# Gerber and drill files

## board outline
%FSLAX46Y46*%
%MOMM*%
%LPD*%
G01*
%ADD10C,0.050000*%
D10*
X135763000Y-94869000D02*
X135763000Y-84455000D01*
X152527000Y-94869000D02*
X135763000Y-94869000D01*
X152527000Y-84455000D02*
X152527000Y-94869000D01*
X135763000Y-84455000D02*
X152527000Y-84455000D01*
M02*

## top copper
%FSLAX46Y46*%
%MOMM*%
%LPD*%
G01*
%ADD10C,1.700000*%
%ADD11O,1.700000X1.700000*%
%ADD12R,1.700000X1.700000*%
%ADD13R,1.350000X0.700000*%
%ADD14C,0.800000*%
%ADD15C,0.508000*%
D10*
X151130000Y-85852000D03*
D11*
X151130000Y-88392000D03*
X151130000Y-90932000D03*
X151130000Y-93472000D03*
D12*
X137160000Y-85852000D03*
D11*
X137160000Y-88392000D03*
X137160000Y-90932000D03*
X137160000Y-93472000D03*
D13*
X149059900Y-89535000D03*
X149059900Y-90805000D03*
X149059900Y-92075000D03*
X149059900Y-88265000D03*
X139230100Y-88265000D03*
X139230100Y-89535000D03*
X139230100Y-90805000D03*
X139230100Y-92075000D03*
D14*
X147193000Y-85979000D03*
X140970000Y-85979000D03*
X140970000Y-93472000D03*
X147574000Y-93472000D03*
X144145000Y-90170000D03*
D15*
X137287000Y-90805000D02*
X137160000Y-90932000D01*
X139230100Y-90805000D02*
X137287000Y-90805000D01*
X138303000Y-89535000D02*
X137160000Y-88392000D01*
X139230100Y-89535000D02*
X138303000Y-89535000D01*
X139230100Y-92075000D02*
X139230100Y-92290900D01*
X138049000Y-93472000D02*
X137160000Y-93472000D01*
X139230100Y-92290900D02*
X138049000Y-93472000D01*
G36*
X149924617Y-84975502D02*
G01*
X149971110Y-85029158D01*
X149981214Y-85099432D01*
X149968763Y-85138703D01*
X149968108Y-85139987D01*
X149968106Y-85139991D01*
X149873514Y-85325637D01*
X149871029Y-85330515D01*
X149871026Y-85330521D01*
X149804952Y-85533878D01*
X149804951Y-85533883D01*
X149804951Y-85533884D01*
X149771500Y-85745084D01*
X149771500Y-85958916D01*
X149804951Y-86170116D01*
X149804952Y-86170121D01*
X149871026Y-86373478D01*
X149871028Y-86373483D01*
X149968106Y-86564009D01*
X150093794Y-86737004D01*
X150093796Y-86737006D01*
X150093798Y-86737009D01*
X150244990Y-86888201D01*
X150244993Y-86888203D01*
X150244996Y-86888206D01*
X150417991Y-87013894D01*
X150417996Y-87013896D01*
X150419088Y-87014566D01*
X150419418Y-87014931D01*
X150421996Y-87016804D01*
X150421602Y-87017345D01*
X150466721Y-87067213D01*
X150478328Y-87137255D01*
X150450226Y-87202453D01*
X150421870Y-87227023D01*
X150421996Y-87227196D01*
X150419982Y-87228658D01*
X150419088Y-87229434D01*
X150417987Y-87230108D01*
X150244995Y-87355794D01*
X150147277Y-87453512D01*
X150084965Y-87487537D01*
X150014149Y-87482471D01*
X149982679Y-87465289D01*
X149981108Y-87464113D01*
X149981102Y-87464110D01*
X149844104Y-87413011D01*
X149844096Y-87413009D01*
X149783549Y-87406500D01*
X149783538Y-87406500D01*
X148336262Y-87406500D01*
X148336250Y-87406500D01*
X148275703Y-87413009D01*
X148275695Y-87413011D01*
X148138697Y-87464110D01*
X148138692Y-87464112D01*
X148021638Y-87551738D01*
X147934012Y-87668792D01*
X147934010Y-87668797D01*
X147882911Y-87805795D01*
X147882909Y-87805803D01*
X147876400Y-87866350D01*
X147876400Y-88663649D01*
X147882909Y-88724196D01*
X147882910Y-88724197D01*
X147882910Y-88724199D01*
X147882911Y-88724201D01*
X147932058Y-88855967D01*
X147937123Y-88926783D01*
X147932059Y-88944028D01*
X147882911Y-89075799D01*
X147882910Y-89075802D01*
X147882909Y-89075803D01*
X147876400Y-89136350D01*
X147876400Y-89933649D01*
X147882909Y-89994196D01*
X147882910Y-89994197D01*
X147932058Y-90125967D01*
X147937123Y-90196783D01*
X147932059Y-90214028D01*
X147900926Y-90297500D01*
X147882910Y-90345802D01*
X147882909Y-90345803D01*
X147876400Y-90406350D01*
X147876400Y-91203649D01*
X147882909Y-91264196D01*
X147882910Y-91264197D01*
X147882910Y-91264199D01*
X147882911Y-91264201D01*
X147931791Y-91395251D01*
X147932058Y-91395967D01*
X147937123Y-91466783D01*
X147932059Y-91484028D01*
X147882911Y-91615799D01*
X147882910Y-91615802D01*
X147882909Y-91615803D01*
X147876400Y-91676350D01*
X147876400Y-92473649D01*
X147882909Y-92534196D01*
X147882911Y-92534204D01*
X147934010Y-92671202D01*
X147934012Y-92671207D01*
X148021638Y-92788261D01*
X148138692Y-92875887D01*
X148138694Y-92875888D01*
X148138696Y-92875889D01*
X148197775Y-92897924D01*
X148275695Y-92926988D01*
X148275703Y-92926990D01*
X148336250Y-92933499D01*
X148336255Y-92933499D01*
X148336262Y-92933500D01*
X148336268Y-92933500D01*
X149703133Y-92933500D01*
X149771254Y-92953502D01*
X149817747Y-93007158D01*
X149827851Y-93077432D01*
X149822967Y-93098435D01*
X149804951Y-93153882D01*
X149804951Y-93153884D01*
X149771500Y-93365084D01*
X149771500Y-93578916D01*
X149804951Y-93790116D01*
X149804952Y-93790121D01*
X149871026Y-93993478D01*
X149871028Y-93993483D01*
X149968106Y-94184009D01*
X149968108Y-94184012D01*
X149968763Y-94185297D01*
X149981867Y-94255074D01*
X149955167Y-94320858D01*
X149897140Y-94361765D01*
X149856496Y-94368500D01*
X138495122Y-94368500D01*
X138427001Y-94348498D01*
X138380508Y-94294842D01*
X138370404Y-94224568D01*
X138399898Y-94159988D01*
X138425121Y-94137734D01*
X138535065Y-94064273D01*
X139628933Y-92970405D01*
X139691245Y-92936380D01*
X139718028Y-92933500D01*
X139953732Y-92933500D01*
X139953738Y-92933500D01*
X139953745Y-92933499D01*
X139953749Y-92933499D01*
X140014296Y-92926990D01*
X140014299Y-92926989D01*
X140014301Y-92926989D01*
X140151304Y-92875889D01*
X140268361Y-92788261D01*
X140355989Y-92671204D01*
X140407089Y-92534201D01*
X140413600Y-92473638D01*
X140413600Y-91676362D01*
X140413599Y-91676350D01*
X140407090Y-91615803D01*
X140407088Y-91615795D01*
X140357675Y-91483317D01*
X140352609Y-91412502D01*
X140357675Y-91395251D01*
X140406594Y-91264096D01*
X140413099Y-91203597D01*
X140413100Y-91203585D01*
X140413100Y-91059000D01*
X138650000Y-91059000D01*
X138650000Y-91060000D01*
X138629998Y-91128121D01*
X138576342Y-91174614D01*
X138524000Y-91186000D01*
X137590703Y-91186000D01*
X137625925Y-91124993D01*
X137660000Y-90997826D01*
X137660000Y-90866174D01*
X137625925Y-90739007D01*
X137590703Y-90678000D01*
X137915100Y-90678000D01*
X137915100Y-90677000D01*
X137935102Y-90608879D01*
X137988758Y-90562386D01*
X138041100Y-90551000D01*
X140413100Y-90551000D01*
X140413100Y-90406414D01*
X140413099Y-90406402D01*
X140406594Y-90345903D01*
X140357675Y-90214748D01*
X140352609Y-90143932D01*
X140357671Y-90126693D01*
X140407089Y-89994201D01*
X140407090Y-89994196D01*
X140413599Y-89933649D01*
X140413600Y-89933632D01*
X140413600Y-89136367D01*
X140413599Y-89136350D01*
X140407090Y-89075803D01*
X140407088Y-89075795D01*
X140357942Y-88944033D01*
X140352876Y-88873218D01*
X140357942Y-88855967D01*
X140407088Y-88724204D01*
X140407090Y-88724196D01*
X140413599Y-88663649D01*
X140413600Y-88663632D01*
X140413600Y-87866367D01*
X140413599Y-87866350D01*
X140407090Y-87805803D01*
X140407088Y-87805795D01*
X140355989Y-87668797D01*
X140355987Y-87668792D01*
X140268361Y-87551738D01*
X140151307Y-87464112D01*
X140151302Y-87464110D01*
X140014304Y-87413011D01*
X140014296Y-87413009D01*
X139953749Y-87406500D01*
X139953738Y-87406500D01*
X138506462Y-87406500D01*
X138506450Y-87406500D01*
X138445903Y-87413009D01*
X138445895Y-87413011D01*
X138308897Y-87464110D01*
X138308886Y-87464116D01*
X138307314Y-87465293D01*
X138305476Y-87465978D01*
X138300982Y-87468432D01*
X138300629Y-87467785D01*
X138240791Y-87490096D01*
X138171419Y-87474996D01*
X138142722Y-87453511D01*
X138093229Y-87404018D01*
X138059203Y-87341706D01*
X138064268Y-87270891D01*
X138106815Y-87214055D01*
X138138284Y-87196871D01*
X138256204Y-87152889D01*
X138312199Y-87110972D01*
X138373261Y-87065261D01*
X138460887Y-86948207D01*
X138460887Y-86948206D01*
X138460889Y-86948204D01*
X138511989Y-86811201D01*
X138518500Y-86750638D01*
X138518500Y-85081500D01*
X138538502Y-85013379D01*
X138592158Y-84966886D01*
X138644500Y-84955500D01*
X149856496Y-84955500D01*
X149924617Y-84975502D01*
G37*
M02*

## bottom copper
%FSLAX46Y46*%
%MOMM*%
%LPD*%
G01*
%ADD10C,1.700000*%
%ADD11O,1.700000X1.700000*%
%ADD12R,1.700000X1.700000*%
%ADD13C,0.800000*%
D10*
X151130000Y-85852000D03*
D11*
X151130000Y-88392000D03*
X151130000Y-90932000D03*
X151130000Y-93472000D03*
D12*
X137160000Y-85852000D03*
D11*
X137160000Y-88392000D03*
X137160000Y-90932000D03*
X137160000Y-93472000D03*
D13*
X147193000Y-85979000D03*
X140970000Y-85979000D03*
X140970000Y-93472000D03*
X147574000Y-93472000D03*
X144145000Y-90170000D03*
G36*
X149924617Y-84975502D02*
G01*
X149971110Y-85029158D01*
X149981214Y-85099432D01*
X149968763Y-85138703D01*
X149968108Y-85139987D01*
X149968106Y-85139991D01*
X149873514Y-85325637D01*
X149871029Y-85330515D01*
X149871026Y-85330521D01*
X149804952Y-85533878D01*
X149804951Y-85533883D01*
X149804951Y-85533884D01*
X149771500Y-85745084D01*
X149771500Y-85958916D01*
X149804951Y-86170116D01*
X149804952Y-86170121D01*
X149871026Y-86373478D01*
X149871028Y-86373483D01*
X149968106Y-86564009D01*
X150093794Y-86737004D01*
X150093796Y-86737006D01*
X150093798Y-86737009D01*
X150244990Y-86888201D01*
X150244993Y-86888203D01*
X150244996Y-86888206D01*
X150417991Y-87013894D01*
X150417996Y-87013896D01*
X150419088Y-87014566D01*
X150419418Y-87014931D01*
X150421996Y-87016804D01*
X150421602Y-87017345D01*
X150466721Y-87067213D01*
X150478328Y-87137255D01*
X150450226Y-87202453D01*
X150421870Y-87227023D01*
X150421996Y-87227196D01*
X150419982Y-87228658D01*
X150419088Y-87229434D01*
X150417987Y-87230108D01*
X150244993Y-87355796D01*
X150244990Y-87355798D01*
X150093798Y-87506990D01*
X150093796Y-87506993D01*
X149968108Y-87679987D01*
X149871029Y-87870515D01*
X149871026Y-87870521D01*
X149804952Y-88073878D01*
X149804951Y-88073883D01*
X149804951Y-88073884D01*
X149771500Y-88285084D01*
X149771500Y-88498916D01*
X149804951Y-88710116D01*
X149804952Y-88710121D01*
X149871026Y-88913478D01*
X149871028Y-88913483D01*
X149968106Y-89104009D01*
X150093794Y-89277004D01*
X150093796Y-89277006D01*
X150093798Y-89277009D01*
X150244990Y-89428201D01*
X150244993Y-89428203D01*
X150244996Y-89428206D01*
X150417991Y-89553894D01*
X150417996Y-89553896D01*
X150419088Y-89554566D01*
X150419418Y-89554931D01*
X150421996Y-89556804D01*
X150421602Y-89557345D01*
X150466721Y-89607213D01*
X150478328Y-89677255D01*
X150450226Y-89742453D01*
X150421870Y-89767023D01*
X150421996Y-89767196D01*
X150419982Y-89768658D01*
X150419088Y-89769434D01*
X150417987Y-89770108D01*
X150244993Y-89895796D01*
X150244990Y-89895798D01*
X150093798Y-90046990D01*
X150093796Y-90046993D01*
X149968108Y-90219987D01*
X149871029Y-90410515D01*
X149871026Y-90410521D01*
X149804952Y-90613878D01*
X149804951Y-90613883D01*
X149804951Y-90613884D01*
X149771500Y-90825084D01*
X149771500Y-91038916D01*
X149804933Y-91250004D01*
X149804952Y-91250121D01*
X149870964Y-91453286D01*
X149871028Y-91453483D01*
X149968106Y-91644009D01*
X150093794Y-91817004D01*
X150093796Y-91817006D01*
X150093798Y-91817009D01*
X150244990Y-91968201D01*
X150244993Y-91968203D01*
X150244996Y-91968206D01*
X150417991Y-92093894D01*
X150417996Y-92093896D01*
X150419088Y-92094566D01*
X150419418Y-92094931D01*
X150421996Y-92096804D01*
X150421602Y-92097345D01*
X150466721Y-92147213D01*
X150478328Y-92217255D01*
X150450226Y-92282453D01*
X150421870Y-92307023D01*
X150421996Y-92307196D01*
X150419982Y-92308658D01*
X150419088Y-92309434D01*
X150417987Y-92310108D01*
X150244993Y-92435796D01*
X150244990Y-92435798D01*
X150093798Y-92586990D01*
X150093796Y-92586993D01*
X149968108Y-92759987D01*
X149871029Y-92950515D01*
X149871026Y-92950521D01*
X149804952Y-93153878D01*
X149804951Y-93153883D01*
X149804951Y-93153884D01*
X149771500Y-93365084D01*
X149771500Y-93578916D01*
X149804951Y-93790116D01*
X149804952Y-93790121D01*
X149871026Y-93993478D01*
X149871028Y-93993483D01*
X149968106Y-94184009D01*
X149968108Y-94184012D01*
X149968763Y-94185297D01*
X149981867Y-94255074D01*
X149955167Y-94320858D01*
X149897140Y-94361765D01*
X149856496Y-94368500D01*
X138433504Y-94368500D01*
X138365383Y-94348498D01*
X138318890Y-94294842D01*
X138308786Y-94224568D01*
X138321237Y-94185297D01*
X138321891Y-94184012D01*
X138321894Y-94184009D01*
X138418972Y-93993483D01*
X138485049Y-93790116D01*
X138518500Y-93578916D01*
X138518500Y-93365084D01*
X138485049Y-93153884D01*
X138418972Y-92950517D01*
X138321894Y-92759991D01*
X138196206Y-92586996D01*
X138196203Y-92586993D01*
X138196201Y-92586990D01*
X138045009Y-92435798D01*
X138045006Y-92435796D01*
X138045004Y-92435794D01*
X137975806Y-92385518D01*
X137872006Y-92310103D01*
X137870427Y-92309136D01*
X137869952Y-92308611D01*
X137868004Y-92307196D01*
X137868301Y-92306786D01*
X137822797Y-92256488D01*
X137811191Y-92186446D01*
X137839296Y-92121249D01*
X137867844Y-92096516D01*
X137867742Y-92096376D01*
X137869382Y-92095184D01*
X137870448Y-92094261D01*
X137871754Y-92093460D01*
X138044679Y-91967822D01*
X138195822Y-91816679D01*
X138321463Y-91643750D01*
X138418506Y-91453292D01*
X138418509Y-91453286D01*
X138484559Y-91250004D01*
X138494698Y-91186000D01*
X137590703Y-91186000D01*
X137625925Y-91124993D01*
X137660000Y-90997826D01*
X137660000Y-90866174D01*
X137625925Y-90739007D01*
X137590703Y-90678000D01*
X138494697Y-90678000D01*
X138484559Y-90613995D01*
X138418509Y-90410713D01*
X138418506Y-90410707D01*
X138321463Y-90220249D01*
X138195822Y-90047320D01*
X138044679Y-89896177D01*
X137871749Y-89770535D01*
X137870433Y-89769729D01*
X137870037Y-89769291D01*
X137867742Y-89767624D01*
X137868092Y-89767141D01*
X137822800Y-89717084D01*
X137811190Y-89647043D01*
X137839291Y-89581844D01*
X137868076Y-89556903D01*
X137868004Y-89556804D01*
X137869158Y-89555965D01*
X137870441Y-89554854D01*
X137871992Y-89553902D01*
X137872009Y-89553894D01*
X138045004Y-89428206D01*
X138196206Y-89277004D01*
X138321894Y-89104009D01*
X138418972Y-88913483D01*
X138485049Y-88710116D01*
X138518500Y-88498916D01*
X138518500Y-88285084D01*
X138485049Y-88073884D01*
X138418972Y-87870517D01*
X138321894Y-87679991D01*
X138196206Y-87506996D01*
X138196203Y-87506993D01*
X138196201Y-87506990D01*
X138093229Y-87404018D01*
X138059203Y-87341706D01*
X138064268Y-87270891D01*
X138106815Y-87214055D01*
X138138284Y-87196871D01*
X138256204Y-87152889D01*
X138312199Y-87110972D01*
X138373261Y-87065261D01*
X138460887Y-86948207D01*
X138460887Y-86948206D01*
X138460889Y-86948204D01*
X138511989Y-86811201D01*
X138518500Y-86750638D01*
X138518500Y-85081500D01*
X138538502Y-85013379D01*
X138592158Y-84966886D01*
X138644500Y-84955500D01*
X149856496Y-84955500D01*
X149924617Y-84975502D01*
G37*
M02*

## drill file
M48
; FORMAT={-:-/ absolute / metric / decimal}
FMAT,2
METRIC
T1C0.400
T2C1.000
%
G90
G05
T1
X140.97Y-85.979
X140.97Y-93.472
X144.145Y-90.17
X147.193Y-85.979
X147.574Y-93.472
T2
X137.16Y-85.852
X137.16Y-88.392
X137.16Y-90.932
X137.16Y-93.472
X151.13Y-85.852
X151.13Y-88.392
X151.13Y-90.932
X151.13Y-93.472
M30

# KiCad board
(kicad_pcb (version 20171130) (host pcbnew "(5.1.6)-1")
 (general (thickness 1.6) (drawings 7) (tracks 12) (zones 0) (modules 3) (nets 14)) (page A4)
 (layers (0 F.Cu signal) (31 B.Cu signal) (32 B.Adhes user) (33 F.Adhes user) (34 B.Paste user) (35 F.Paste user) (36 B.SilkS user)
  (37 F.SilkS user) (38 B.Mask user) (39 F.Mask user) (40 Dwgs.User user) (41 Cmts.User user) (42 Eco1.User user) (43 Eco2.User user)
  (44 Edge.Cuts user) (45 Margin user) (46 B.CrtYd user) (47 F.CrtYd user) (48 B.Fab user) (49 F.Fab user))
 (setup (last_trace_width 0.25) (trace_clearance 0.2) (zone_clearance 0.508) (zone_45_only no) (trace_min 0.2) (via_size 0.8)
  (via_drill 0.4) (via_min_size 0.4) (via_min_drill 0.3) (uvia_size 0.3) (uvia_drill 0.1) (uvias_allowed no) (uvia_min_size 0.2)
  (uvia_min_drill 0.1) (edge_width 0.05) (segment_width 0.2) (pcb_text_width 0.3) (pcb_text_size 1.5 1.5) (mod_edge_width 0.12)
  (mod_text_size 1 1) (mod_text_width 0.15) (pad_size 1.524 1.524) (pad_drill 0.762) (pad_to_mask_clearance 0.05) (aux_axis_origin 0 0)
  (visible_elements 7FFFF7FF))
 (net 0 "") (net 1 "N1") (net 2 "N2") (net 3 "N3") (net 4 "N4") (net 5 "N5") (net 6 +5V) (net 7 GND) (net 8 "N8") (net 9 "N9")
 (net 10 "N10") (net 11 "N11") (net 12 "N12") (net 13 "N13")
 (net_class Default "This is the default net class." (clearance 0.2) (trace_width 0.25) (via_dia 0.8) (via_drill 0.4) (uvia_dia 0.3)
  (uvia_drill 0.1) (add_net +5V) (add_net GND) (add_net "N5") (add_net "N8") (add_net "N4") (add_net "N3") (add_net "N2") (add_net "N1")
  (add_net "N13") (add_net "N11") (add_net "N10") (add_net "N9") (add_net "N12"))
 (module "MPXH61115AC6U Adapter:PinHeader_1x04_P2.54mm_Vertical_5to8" (layer F.Cu) (at 151.13 85.852)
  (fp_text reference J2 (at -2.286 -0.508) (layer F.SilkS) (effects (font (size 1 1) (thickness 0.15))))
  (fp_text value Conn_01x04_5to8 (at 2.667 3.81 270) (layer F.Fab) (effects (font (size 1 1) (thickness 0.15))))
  (pad 8 thru_hole circle (at 0 0) (size 1.7 1.7) (drill 1) (layers *.Cu *.Mask) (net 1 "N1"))
  (pad 7 thru_hole oval (at 0 2.54) (size 1.7 1.7) (drill 1) (layers *.Cu *.Mask) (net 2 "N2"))
  (pad 6 thru_hole oval (at 0 5.08) (size 1.7 1.7) (drill 1) (layers *.Cu *.Mask) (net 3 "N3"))
  (pad 5 thru_hole oval (at 0 7.62) (size 1.7 1.7) (drill 1) (layers *.Cu *.Mask) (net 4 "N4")))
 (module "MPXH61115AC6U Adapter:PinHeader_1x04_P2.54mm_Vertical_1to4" (layer F.Cu) (at 137.16 85.852)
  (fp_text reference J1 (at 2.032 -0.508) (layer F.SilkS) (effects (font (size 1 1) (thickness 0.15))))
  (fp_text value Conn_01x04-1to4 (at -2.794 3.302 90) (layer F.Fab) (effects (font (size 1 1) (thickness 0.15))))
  (pad 1 thru_hole rect (at 0 0) (size 1.7 1.7) (drill 1) (layers *.Cu *.Mask) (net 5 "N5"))
  (pad 2 thru_hole oval (at 0 2.54) (size 1.7 1.7) (drill 1) (layers *.Cu *.Mask) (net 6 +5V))
  (pad 3 thru_hole oval (at 0 5.08) (size 1.7 1.7) (drill 1) (layers *.Cu *.Mask) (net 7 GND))
  (pad 4 thru_hole oval (at 0 7.62) (size 1.7 1.7) (drill 1) (layers *.Cu *.Mask) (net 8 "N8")))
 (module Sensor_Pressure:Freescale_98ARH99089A (layer F.Cu) (at 144.145 90.17)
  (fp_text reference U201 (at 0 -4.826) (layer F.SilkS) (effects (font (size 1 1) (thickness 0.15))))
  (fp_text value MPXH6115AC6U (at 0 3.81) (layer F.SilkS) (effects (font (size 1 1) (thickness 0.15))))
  (pad 7 smd rect (at 4.9149 -0.635) (size 1.35 0.7) (layers F.Cu F.Paste F.Mask) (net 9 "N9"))
  (pad 6 smd rect (at 4.9149 0.635) (size 1.35 0.7) (layers F.Cu F.Paste F.Mask) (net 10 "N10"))
  (pad 5 smd rect (at 4.9149 1.905) (size 1.35 0.7) (layers F.Cu F.Paste F.Mask) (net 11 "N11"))
  (pad 8 smd rect (at 4.9149 -1.905) (size 1.35 0.7) (layers F.Cu F.Paste F.Mask) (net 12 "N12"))
  (pad 1 smd rect (at -4.9149 -1.905) (size 1.35 0.7) (layers F.Cu F.Paste F.Mask) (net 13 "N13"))
  (pad 2 smd rect (at -4.9149 -0.635) (size 1.35 0.7) (layers F.Cu F.Paste F.Mask) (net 6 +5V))
  (pad 3 smd rect (at -4.9149 0.635) (size 1.35 0.7) (layers F.Cu F.Paste F.Mask) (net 7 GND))
  (pad 4 smd rect (at -4.9149 1.905) (size 1.35 0.7) (layers F.Cu F.Paste F.Mask) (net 8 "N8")))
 (gr_line (start 135.763 94.869) (end 135.763 84.455) (layer Edge.Cuts) (width 0.05))
 (gr_line (start 152.527 94.869) (end 135.763 94.869) (layer Edge.Cuts) (width 0.05))
 (gr_line (start 152.527 84.455) (end 152.527 94.869) (layer Edge.Cuts) (width 0.05))
 (gr_line (start 135.763 84.455) (end 152.527 84.455) (layer Edge.Cuts) (width 0.05))
 (via (at 147.193 85.979) (size 0.8) (drill 0.4) (layers F.Cu B.Cu) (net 7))
 (via (at 140.97 85.979) (size 0.8) (drill 0.4) (layers F.Cu B.Cu) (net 7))
 (via (at 140.97 93.472) (size 0.8) (drill 0.4) (layers F.Cu B.Cu) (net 7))
 (via (at 147.574 93.472) (size 0.8) (drill 0.4) (layers F.Cu B.Cu) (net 7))
 (via (at 144.145 90.17) (size 0.8) (drill 0.4) (layers F.Cu B.Cu) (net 7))
 (segment (start 137.287 90.805) (end 137.16 90.932) (width 0.508) (layer F.Cu) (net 7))
 (segment (start 139.2301 90.805) (end 137.287 90.805) (width 0.508) (layer F.Cu) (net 7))
 (segment (start 138.303 89.535) (end 137.16 88.392) (width 0.508) (layer F.Cu) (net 6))
 (segment (start 139.2301 89.535) (end 138.303 89.535) (width 0.508) (layer F.Cu) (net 6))
 (segment (start 139.2301 92.075) (end 139.2301 92.2909) (width 0.508) (layer F.Cu) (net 8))
 (segment (start 138.049 93.472) (end 137.16 93.472) (width 0.508) (layer F.Cu) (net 8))
 (segment (start 139.2301 92.2909) (end 138.049 93.472) (width 0.508) (layer F.Cu) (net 8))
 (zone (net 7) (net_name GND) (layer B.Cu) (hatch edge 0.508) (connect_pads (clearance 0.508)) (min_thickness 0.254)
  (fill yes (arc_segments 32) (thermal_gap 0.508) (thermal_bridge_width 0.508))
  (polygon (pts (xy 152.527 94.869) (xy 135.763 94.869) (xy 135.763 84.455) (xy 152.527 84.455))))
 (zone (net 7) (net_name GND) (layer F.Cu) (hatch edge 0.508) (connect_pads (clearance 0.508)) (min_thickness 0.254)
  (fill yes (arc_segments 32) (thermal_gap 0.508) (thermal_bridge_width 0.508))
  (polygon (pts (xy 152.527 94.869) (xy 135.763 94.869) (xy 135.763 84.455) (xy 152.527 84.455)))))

